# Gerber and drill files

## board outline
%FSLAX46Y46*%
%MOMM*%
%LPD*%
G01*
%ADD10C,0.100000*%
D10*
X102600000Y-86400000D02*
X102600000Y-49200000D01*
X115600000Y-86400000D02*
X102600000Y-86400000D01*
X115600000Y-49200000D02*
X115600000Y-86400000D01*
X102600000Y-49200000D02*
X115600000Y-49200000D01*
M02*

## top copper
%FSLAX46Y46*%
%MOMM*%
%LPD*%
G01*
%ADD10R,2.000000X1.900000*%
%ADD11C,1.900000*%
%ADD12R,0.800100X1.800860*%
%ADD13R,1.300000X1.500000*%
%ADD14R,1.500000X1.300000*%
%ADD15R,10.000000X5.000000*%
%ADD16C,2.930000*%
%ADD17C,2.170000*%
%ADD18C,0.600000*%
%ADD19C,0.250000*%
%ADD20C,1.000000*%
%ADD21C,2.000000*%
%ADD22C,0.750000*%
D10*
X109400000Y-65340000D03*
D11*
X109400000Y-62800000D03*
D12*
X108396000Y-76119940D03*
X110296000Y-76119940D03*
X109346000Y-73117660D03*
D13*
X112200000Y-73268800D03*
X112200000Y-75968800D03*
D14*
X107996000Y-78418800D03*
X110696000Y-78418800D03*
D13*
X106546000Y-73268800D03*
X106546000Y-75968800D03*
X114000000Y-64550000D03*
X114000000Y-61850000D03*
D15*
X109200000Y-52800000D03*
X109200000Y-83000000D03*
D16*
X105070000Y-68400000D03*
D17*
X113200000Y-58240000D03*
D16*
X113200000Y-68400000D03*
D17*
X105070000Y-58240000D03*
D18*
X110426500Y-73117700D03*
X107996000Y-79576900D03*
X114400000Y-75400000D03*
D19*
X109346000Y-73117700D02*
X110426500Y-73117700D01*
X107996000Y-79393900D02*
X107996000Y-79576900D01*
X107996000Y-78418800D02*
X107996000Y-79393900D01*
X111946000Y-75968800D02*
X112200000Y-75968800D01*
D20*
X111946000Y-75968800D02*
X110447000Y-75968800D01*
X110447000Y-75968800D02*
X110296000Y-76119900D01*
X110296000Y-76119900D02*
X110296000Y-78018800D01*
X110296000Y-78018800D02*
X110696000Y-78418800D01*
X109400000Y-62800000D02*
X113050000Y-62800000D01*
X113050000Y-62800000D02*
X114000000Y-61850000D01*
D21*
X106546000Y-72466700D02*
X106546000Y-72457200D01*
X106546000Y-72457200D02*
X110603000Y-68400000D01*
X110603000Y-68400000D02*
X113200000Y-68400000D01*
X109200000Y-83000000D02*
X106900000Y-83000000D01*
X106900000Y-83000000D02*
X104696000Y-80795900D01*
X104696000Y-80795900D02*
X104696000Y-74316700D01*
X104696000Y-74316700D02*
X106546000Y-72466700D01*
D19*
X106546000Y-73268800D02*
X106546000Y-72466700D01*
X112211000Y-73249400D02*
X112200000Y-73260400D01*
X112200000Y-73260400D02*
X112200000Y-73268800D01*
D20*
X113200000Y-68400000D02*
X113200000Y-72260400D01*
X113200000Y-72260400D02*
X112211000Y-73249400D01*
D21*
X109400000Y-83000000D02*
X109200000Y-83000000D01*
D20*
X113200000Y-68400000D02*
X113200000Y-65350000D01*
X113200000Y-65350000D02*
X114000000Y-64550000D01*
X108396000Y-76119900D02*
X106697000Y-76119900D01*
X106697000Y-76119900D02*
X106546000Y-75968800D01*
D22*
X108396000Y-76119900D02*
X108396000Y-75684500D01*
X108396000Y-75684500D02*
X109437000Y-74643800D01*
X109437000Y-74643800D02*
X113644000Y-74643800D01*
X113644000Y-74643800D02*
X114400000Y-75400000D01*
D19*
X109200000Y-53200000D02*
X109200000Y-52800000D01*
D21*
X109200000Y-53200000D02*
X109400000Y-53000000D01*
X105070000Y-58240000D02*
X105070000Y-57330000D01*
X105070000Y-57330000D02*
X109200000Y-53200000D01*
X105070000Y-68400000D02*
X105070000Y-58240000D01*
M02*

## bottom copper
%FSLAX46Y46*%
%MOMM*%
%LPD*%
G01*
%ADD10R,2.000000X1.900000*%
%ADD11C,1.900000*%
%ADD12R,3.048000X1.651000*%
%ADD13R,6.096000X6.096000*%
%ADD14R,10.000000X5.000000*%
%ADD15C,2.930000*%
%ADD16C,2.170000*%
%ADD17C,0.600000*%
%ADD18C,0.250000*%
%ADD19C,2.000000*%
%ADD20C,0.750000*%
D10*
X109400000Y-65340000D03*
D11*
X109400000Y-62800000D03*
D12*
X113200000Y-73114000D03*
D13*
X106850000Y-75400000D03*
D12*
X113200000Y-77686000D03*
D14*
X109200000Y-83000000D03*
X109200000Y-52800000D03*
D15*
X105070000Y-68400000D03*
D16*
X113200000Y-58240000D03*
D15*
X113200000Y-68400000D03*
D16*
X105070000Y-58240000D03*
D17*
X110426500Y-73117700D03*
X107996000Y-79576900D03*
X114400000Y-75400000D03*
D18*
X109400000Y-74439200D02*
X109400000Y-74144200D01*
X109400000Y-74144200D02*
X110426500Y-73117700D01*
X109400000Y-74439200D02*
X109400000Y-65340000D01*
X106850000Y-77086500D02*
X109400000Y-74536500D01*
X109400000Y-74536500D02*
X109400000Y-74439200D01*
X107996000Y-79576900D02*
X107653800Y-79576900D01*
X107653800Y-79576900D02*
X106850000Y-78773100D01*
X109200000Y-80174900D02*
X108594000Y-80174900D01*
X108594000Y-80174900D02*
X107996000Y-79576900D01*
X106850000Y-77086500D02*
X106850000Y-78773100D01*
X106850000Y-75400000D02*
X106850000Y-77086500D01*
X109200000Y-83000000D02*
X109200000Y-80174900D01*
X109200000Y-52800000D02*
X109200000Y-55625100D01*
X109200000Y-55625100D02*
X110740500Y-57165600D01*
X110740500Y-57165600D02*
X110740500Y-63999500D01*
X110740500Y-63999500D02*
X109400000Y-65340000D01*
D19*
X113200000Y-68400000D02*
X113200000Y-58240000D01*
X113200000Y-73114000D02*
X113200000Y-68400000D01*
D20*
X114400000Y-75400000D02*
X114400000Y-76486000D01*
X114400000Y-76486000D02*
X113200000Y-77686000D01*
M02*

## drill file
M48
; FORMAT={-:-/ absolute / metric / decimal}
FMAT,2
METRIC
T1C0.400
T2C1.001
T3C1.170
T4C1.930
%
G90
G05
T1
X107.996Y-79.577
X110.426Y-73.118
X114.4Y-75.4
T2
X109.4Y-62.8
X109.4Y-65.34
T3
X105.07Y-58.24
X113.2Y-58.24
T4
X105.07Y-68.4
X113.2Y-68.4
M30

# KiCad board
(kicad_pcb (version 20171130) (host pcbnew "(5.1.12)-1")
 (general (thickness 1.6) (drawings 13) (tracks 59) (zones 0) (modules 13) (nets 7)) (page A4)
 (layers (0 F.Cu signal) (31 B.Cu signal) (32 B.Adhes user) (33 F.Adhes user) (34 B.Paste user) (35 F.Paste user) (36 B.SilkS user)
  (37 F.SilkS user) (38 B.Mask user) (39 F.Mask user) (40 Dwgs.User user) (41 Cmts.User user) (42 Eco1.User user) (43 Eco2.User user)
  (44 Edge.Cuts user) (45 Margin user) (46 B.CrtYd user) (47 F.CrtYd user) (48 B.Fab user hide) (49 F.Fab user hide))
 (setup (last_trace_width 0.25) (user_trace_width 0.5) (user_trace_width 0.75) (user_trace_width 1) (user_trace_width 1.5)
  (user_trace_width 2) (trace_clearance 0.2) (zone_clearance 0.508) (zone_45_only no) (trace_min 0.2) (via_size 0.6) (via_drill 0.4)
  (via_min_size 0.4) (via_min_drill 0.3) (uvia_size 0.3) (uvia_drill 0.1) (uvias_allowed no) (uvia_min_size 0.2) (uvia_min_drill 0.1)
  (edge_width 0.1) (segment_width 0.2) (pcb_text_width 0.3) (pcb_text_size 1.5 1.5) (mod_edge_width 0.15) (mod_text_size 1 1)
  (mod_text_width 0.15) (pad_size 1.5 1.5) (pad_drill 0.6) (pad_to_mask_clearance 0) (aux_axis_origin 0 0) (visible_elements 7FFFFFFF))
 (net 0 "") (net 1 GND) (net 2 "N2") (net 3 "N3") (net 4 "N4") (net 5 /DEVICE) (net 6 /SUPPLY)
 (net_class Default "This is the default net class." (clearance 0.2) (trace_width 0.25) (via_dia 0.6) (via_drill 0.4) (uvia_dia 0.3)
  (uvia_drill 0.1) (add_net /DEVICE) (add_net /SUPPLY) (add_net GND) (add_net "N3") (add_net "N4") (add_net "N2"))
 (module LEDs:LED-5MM (layer F.Cu) (at 109.4 65.34 90)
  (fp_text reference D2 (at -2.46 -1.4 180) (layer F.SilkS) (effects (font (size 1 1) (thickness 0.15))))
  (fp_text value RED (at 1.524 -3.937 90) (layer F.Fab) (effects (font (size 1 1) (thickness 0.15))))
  (pad 1 thru_hole rect (at 0 0 180) (size 2 1.9) (drill 1.00076) (layers *.Cu *.Mask F.SilkS) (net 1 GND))
  (pad 2 thru_hole circle (at 2.54 0 90) (size 1.9 1.9) (drill 1.00076) (layers *.Cu *.Mask F.SilkS) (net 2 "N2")))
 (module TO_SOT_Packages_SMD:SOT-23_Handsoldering (layer F.Cu) (at 109.346 74.6188)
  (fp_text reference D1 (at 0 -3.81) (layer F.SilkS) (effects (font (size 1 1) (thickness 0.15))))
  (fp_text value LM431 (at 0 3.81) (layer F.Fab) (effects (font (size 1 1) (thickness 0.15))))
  (pad 1 smd rect (at -0.95 1.50114) (size 0.8001 1.80086) (layers F.Cu F.Paste F.Mask) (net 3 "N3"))
  (pad 2 smd rect (at 0.95 1.50114) (size 0.8001 1.80086) (layers F.Cu F.Paste F.Mask) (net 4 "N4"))
  (pad 3 smd rect (at 0 -1.50114) (size 0.8001 1.80086) (layers F.Cu F.Paste F.Mask) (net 1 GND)))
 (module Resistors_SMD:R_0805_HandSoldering (layer F.Cu) (at 112.2 74.6188 270)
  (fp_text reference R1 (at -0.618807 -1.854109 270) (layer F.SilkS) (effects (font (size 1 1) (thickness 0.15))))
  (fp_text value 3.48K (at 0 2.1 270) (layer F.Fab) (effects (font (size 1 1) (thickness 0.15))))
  (pad 1 smd rect (at -1.35 0 270) (size 1.5 1.3) (layers F.Cu F.Paste F.Mask) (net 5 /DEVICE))
  (pad 2 smd rect (at 1.35 0 270) (size 1.5 1.3) (layers F.Cu F.Paste F.Mask) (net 4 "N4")))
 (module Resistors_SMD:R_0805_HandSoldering (layer F.Cu) (at 109.346 78.4188)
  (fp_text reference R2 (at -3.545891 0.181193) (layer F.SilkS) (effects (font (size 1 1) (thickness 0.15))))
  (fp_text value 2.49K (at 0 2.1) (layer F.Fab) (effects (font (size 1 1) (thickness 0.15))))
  (pad 1 smd rect (at -1.35 0) (size 1.5 1.3) (layers F.Cu F.Paste F.Mask) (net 1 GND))
  (pad 2 smd rect (at 1.35 0) (size 1.5 1.3) (layers F.Cu F.Paste F.Mask) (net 4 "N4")))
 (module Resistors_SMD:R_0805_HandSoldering (layer F.Cu) (at 106.546 74.6188 270)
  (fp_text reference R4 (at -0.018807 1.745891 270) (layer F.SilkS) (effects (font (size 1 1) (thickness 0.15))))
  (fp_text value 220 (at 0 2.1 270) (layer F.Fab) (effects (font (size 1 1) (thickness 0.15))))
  (pad 1 smd rect (at -1.35 0 270) (size 1.5 1.3) (layers F.Cu F.Paste F.Mask) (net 5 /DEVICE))
  (pad 2 smd rect (at 1.35 0 270) (size 1.5 1.3) (layers F.Cu F.Paste F.Mask) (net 3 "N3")))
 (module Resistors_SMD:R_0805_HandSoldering (layer F.Cu) (at 114 63.2 90)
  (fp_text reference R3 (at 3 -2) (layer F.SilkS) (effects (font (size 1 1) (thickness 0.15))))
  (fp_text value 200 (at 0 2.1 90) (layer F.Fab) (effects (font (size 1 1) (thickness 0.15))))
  (pad 1 smd rect (at -1.35 0 90) (size 1.5 1.3) (layers F.Cu F.Paste F.Mask) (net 5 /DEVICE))
  (pad 2 smd rect (at 1.35 0 90) (size 1.5 1.3) (layers F.Cu F.Paste F.Mask) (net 2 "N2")))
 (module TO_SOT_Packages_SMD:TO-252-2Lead (layer B.Cu) (at 113.2 75.4 270)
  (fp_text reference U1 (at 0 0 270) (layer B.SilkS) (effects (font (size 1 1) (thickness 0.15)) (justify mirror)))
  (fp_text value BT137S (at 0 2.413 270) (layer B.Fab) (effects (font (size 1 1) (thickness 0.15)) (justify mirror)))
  (pad 1 smd rect (at -2.286 0 270) (size 1.651 3.048) (layers B.Cu B.Paste B.Mask) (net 5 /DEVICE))
  (pad 2 smd rect (at 0 6.35 270) (size 6.096 6.096) (layers B.Cu B.Paste B.Mask) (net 1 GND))
  (pad 3 smd rect (at 2.286 0 270) (size 1.651 3.048) (layers B.Cu B.Paste B.Mask) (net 3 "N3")))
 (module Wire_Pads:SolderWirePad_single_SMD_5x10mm (layer F.Cu) (at 109.2 52.8 90)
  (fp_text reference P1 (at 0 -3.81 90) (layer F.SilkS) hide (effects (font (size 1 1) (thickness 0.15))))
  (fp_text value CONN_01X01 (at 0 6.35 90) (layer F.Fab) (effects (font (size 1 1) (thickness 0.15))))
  (pad 1 smd rect (at 0 0 90) (size 5 10) (layers F.Cu F.Paste F.Mask) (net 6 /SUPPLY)))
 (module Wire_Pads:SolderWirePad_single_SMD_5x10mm (layer F.Cu) (at 109.2 83 90)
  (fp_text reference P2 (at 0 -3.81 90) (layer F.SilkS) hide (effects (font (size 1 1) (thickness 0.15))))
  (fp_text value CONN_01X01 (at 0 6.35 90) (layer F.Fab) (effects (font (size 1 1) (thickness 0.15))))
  (pad 1 smd rect (at 0 0 90) (size 5 10) (layers F.Cu F.Paste F.Mask) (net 5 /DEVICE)))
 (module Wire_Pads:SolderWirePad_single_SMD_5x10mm (layer B.Cu) (at 109.2 83 90)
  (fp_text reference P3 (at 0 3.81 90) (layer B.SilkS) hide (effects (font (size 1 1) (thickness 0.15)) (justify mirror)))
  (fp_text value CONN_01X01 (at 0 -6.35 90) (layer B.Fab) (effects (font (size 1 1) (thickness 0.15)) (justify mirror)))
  (pad 1 smd rect (at 0 0 90) (size 5 10) (layers B.Cu B.Paste B.Mask) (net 1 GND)))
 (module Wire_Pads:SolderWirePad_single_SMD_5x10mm (layer B.Cu) (at 109.2 52.8 90)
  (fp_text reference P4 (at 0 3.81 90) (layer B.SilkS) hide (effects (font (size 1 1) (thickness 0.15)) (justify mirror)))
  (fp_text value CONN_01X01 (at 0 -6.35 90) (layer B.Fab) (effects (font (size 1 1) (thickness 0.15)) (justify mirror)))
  (pad 1 smd rect (at 0 0 90) (size 5 10) (layers B.Cu B.Paste B.Mask) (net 1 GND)))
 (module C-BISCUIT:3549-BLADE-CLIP (layer B.Cu) (at 109.135 63.32)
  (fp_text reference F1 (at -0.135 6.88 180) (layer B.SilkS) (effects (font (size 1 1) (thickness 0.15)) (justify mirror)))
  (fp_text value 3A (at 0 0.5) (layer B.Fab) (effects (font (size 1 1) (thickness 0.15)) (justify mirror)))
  (pad 1 thru_hole circle (at -4.065 5.08) (size 2.93 2.93) (drill 1.93) (layers *.Cu *.Mask B.SilkS) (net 6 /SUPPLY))
  (pad 2 thru_hole circle (at 4.065 -5.08) (size 2.17 2.17) (drill 1.17) (layers *.Cu *.Mask B.SilkS) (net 5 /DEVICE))
  (pad 2 thru_hole circle (at 4.065 5.08) (size 2.93 2.93) (drill 1.93) (layers *.Cu *.Mask B.SilkS) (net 5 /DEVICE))
  (pad 1 thru_hole circle (at -4.065 -5.08) (size 2.17 2.17) (drill 1.17) (layers *.Cu *.Mask B.SilkS) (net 6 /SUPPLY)))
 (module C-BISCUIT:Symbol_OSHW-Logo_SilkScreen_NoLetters (layer B.Cu) (at 105.8 63.2 270)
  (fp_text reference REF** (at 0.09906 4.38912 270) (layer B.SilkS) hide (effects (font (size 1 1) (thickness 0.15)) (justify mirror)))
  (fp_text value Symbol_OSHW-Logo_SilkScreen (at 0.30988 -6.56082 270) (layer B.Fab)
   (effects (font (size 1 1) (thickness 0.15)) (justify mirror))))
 (gr_line (start 102.6 86.4) (end 102.6 49.2) (layer Edge.Cuts) (width 0.1))
 (gr_line (start 115.6 86.4) (end 102.6 86.4) (layer Edge.Cuts) (width 0.1))
 (gr_line (start 115.6 49.2) (end 115.6 86.4) (layer Edge.Cuts) (width 0.1))
 (gr_line (start 102.6 49.2) (end 115.6 49.2) (layer Edge.Cuts) (width 0.1))
 (segment (start 109.346 73.1177) (end 110.4265 73.1177) (width 0.25) (layer F.Cu) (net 1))
 (segment (start 109.4 74.4392) (end 109.4 74.1442) (width 0.25) (layer B.Cu) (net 1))
 (segment (start 109.4 74.1442) (end 110.4265 73.1177) (width 0.25) (layer B.Cu) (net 1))
 (segment (start 109.4 74.4392) (end 109.4 65.34) (width 0.25) (layer B.Cu) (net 1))
 (segment (start 106.85 77.0865) (end 109.4 74.5365) (width 0.25) (layer B.Cu) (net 1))
 (segment (start 109.4 74.5365) (end 109.4 74.4392) (width 0.25) (layer B.Cu) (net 1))
 (segment (start 107.996 79.5769) (end 107.6538 79.5769) (width 0.25) (layer B.Cu) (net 1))
 (segment (start 107.6538 79.5769) (end 106.85 78.7731) (width 0.25) (layer B.Cu) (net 1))
 (segment (start 109.2 80.1749) (end 108.594 80.1749) (width 0.25) (layer B.Cu) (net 1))
 (segment (start 108.594 80.1749) (end 107.996 79.5769) (width 0.25) (layer B.Cu) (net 1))
 (segment (start 107.996 79.3939) (end 107.996 79.5769) (width 0.25) (layer F.Cu) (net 1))
 (segment (start 107.996 78.4188) (end 107.996 79.3939) (width 0.25) (layer F.Cu) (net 1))
 (segment (start 106.85 77.0865) (end 106.85 78.7731) (width 0.25) (layer B.Cu) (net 1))
 (segment (start 106.85 75.4) (end 106.85 77.0865) (width 0.25) (layer B.Cu) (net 1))
 (segment (start 109.2 83) (end 109.2 80.1749) (width 0.25) (layer B.Cu) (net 1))
 (segment (start 109.2 52.8) (end 109.2 55.6251) (width 0.25) (layer B.Cu) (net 1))
 (segment (start 109.2 55.6251) (end 110.7405 57.1656) (width 0.25) (layer B.Cu) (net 1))
 (segment (start 110.7405 57.1656) (end 110.7405 63.9995) (width 0.25) (layer B.Cu) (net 1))
 (segment (start 110.7405 63.9995) (end 109.4 65.34) (width 0.25) (layer B.Cu) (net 1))
 (via (at 110.4265 73.1177) (size 0.6) (layers F.Cu B.Cu) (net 1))
 (via (at 107.996 79.5769) (size 0.6) (layers F.Cu B.Cu) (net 1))
 (segment (start 111.946 75.9688) (end 112.2 75.9688) (width 0.25) (layer F.Cu) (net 4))
 (segment (start 111.946 75.9688) (end 110.447 75.9688) (width 1) (layer F.Cu) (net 4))
 (segment (start 110.447 75.9688) (end 110.296 76.1199) (width 1) (layer F.Cu) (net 4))
 (segment (start 110.296 76.1199) (end 110.296 78.0188) (width 1) (layer F.Cu) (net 4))
 (segment (start 110.296 78.0188) (end 110.696 78.4188) (width 1) (layer F.Cu) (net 4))
 (segment (start 109.4 62.8) (end 113.05 62.8) (width 1) (layer F.Cu) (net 2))
 (segment (start 113.05 62.8) (end 114 61.85) (width 1) (layer F.Cu) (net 2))
 (segment (start 106.546 72.4667) (end 106.546 72.4572) (width 2) (layer F.Cu) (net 5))
 (segment (start 106.546 72.4572) (end 110.603 68.4) (width 2) (layer F.Cu) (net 5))
 (segment (start 110.603 68.4) (end 113.2 68.4) (width 2) (layer F.Cu) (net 5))
 (segment (start 109.2 83) (end 106.9 83) (width 2) (layer F.Cu) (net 5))
 (segment (start 106.9 83) (end 104.696 80.7959) (width 2) (layer F.Cu) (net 5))
 (segment (start 104.696 80.7959) (end 104.696 74.3167) (width 2) (layer F.Cu) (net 5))
 (segment (start 104.696 74.3167) (end 106.546 72.4667) (width 2) (layer F.Cu) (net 5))
 (segment (start 106.546 73.2688) (end 106.546 72.4667) (width 0.25) (layer F.Cu) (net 5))
 (segment (start 112.211 73.2494) (end 112.2 73.2604) (width 0.25) (layer F.Cu) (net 5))
 (segment (start 112.2 73.2604) (end 112.2 73.2688) (width 0.25) (layer F.Cu) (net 5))
 (segment (start 113.2 68.4) (end 113.2 72.2604) (width 1) (layer F.Cu) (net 5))
 (segment (start 113.2 72.2604) (end 112.211 73.2494) (width 1) (layer F.Cu) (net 5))
 (segment (start 109.4 83) (end 109.2 83) (width 2) (layer F.Cu) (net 5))
 (segment (start 113.2 68.4) (end 113.2 58.24) (width 2) (layer B.Cu) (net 5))
 (segment (start 113.2 68.4) (end 113.2 65.35) (width 1) (layer F.Cu) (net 5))
 (segment (start 113.2 65.35) (end 114 64.55) (width 1) (layer F.Cu) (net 5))
 (segment (start 113.2 73.114) (end 113.2 68.4) (width 2) (layer B.Cu) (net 5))
 (segment (start 114.4 75.4) (end 114.4 76.486) (width 0.75) (layer B.Cu) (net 3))
 (segment (start 114.4 76.486) (end 113.2 77.686) (width 0.75) (layer B.Cu) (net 3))
 (segment (start 108.396 76.1199) (end 106.697 76.1199) (width 1) (layer F.Cu) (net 3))
 (segment (start 106.697 76.1199) (end 106.546 75.9688) (width 1) (layer F.Cu) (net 3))
 (segment (start 108.396 76.1199) (end 108.396 75.6845) (width 0.75) (layer F.Cu) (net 3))
 (segment (start 108.396 75.6845) (end 109.437 74.6438) (width 0.75) (layer F.Cu) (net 3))
 (segment (start 109.437 74.6438) (end 113.644 74.6438) (width 0.75) (layer F.Cu) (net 3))
 (segment (start 113.644 74.6438) (end 114.4 75.4) (width 0.75) (layer F.Cu) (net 3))
 (via (at 114.4 75.4) (size 0.6) (layers F.Cu B.Cu) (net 3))
 (segment (start 109.2 53.2) (end 109.2 52.8) (width 0.25) (layer F.Cu) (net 6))
 (segment (start 109.2 53.2) (end 109.4 53) (width 2) (layer F.Cu) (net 6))
 (segment (start 105.07 58.24) (end 105.07 57.33) (width 2) (layer F.Cu) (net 6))
 (segment (start 105.07 57.33) (end 109.2 53.2) (width 2) (layer F.Cu) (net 6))
 (segment (start 105.07 68.4) (end 105.07 58.24) (width 2) (layer F.Cu) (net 6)))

